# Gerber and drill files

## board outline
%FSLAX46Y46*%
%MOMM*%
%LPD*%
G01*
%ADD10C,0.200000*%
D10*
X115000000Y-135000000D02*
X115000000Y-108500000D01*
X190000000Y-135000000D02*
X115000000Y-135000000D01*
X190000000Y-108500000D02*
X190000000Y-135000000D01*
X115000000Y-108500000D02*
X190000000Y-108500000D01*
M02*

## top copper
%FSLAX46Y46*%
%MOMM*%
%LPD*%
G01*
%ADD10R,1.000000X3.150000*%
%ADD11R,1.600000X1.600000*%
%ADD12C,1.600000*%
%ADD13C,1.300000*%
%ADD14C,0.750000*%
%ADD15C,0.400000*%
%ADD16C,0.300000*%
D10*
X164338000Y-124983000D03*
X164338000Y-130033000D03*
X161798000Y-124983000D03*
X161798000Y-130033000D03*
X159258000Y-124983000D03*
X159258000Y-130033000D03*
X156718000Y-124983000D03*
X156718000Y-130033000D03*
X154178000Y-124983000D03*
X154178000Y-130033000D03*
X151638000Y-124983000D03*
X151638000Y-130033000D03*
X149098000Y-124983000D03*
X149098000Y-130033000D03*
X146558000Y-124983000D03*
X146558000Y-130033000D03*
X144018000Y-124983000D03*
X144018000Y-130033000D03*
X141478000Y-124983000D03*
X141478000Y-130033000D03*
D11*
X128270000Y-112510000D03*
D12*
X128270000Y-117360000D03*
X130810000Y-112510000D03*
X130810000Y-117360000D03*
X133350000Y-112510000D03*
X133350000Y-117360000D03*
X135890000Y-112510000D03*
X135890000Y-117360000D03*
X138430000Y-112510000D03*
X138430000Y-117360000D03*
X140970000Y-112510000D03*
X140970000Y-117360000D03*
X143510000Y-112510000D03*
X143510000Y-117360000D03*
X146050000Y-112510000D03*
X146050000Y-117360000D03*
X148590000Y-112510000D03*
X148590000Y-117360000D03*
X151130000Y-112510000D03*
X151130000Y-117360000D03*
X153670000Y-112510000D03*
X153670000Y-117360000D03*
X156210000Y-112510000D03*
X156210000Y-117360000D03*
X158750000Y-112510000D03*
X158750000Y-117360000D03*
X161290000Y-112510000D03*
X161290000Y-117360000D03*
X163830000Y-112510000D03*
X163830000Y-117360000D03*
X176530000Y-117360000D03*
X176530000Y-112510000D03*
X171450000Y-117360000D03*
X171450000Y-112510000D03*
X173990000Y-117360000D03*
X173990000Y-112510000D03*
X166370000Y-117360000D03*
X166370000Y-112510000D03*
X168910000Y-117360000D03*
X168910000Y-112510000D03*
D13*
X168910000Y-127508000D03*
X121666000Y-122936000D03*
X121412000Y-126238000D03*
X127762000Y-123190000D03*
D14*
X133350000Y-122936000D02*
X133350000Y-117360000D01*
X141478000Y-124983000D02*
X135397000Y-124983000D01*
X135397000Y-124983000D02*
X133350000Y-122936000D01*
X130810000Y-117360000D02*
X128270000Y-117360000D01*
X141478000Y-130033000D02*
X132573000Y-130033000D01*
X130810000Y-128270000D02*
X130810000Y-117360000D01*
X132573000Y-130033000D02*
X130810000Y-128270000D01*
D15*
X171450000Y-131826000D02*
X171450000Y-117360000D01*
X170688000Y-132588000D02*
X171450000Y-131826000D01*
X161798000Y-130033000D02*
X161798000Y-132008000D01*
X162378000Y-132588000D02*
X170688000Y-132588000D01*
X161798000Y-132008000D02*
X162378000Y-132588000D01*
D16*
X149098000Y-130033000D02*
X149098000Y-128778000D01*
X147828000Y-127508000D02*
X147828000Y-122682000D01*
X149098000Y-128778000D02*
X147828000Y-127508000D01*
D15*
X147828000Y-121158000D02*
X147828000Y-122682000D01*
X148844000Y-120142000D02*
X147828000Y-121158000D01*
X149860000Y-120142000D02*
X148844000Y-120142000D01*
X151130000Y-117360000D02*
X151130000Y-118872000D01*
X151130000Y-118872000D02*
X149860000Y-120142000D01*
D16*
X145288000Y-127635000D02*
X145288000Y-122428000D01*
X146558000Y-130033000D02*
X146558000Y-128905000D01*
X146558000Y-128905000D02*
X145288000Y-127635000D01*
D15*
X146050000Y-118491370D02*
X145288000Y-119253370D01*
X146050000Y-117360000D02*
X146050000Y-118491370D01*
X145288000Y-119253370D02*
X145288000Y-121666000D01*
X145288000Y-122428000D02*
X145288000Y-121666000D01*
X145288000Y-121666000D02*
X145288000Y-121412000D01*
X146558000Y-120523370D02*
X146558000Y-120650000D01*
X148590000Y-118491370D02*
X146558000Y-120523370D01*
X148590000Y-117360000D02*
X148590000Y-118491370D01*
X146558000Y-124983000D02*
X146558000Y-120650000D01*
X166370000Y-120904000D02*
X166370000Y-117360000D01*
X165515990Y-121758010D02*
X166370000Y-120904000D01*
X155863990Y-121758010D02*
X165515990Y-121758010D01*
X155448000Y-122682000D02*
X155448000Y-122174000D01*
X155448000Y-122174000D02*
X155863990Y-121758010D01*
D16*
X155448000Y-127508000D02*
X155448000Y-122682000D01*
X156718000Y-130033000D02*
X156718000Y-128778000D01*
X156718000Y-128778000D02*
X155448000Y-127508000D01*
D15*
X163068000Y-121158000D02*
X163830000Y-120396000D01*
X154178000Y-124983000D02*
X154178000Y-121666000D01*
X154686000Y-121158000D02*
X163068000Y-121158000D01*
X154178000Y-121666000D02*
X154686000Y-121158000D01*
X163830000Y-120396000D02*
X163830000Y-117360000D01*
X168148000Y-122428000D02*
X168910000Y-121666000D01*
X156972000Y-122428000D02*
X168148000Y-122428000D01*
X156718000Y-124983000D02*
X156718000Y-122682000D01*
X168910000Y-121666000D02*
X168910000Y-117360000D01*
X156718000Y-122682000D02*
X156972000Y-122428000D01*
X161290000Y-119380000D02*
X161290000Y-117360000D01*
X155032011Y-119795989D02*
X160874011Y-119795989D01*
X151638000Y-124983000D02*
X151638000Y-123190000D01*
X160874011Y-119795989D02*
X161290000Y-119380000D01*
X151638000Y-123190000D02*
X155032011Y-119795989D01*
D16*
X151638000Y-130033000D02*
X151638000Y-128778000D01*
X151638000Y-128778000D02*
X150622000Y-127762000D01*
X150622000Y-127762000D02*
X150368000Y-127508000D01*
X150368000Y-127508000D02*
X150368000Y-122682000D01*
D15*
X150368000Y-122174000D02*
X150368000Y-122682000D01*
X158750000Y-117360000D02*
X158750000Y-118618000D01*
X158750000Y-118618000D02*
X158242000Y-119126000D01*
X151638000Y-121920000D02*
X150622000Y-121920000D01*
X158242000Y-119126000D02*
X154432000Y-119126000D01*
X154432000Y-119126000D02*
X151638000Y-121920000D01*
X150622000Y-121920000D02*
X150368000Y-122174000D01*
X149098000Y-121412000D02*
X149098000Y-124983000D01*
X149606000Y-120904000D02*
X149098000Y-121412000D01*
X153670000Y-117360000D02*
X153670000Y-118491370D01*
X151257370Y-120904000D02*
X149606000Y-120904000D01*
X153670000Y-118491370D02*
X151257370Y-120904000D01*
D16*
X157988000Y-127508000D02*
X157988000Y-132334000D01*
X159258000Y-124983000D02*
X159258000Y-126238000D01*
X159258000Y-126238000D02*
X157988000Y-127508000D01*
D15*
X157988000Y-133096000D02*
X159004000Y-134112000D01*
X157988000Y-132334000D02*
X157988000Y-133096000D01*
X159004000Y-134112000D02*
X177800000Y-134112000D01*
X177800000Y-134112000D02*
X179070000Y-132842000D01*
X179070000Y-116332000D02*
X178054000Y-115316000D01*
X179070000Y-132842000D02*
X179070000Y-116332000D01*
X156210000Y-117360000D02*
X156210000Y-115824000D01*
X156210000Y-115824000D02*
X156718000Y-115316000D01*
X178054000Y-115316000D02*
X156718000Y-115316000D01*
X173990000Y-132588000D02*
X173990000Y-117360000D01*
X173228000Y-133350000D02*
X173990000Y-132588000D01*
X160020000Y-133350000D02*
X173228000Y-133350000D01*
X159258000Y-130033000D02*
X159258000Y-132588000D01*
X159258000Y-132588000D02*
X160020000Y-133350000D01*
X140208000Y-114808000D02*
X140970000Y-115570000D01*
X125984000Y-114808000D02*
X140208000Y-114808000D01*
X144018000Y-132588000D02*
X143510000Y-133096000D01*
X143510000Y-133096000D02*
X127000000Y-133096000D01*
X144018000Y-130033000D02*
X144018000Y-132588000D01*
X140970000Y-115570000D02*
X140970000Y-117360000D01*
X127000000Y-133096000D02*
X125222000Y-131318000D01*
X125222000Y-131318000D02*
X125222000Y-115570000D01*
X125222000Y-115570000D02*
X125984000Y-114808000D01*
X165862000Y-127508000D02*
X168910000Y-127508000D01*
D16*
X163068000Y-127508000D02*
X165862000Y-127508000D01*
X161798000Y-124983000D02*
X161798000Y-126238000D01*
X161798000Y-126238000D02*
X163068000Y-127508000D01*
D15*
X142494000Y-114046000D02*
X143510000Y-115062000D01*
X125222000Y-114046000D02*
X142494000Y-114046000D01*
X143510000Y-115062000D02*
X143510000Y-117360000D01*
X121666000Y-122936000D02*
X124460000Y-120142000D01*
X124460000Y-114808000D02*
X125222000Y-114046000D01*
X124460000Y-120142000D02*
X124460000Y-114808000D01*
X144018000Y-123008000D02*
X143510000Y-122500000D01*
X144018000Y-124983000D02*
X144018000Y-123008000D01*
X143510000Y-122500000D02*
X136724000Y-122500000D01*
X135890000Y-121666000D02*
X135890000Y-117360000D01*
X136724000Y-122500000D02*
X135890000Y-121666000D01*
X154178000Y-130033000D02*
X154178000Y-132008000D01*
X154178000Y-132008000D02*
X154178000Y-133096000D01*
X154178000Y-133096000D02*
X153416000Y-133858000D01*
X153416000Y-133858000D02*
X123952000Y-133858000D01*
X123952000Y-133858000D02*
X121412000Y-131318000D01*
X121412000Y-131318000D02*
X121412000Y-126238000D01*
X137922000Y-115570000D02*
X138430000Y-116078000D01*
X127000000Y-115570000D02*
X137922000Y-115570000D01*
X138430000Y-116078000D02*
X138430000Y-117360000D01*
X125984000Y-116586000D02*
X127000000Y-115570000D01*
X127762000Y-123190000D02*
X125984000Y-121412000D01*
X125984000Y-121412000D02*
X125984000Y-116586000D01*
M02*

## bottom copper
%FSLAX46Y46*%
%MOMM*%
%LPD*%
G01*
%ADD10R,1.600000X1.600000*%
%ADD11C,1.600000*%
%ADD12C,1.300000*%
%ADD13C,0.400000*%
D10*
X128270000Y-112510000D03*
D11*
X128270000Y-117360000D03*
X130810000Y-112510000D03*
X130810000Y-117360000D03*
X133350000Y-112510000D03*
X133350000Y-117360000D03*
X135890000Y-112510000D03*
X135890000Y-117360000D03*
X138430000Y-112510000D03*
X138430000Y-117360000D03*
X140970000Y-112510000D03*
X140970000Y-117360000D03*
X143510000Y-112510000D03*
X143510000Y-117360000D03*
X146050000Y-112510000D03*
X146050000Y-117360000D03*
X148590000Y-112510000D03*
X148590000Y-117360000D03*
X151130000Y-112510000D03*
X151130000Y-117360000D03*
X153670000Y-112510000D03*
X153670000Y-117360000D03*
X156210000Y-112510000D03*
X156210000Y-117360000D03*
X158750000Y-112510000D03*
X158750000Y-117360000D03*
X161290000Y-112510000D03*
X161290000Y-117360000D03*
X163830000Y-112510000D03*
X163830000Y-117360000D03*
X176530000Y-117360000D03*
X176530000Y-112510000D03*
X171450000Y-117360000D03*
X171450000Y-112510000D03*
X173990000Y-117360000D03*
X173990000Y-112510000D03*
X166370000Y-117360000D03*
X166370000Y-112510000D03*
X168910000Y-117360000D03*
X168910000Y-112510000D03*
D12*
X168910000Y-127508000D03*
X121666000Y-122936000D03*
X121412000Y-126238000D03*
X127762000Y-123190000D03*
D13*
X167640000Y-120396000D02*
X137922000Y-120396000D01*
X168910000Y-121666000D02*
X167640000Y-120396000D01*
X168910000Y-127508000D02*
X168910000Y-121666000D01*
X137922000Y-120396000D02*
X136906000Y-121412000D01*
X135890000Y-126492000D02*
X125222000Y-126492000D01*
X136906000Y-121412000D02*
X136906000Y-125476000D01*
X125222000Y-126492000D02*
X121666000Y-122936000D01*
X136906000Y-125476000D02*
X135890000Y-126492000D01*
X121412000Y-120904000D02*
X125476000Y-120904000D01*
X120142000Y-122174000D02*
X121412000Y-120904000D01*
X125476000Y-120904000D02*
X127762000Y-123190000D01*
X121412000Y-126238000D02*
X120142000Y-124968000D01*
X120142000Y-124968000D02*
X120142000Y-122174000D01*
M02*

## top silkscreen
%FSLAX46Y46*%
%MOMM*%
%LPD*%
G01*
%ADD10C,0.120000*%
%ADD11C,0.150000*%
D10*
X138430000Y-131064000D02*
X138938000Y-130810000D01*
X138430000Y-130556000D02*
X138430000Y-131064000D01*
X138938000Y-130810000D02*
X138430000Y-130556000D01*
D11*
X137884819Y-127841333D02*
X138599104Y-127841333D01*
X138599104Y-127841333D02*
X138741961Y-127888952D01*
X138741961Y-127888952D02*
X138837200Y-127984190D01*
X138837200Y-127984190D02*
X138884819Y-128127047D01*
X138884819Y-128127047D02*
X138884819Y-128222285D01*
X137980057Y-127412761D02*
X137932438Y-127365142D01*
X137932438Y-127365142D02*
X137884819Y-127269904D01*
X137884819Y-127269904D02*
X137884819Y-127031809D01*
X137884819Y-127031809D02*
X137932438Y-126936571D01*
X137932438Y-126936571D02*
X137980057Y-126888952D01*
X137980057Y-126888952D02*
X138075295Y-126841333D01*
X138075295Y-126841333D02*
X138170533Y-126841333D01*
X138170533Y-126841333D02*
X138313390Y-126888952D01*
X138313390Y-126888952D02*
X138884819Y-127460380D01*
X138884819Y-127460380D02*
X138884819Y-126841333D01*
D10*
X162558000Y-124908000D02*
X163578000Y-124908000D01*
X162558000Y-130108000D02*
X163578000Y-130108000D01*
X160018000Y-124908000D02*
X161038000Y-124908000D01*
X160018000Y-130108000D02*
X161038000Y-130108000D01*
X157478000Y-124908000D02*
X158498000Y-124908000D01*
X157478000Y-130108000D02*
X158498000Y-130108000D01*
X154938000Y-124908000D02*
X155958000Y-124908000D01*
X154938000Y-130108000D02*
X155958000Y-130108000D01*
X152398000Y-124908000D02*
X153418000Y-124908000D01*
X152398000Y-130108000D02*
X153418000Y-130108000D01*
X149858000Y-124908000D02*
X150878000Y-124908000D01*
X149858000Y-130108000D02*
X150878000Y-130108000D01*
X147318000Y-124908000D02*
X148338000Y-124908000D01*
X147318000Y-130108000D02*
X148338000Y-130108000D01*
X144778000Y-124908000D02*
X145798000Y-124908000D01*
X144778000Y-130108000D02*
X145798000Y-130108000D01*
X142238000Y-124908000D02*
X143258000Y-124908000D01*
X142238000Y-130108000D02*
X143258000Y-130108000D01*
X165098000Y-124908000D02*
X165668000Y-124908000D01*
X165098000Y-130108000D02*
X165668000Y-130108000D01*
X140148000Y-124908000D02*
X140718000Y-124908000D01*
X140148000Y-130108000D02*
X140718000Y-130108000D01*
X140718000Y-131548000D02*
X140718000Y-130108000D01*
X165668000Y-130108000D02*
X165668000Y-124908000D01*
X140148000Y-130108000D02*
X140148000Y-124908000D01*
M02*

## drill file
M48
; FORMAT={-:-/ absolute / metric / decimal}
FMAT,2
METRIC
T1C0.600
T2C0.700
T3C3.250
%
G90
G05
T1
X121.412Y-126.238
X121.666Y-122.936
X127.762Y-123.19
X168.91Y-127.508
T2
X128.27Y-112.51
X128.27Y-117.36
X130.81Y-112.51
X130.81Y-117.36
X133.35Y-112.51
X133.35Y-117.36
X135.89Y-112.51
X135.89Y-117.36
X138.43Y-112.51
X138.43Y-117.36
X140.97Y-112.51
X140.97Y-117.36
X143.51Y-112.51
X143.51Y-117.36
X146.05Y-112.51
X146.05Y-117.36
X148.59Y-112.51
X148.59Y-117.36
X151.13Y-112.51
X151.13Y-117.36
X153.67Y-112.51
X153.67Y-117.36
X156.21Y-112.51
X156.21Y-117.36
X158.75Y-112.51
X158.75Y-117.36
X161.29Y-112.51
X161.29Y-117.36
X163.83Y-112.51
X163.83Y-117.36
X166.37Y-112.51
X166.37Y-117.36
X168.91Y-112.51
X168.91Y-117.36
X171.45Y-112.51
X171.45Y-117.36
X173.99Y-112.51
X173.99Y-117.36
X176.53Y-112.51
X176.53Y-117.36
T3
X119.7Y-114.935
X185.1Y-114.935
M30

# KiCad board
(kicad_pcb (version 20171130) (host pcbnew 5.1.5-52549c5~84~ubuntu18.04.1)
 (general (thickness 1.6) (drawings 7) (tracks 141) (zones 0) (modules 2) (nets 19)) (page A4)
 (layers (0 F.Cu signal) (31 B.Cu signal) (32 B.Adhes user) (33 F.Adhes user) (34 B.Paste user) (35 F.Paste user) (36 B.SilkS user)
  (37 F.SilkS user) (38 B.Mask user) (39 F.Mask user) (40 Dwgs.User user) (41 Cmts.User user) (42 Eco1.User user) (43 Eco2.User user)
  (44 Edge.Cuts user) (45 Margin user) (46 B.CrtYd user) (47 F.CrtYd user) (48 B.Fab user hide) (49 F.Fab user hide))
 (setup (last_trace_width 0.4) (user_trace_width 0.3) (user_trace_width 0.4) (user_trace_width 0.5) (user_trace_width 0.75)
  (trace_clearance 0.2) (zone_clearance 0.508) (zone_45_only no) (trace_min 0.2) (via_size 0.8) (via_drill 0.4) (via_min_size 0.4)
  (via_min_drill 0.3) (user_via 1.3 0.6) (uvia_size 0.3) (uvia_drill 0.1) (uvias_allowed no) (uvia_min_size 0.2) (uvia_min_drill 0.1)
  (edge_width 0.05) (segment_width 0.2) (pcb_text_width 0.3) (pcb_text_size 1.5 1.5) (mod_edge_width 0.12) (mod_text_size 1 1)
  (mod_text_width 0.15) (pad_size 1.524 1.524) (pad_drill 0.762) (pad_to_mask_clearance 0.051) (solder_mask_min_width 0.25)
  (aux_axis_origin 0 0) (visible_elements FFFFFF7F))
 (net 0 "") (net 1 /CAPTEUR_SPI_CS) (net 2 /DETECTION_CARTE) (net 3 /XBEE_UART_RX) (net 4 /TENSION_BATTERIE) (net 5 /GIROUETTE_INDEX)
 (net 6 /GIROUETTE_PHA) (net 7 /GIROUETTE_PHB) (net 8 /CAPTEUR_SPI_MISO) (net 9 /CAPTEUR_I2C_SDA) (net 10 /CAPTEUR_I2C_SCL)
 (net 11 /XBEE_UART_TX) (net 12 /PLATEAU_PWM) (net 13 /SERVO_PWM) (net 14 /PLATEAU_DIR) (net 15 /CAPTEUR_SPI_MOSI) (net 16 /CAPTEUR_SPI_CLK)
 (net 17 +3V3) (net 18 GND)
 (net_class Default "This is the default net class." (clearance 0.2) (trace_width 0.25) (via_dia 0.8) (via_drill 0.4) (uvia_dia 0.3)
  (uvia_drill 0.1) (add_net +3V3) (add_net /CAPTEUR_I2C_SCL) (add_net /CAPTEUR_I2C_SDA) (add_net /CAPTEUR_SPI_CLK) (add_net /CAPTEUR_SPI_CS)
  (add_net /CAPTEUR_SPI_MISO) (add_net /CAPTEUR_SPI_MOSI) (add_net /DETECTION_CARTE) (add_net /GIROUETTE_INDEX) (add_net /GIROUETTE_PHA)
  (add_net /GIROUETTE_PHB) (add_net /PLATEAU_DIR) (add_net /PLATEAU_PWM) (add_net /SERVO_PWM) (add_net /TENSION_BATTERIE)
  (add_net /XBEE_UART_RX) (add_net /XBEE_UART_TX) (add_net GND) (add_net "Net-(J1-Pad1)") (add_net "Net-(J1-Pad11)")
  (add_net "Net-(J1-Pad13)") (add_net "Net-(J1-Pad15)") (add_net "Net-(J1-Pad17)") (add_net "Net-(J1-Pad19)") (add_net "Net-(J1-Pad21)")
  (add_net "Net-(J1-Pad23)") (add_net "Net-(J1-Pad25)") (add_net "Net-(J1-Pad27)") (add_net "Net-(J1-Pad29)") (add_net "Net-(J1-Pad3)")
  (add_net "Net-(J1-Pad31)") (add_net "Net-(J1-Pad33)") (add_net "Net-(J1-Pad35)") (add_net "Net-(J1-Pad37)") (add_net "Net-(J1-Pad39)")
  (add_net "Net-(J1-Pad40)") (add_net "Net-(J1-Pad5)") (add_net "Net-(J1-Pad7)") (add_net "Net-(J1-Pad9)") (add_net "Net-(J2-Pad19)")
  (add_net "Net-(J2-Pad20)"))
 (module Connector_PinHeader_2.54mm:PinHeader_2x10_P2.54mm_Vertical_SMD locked (layer F.Cu) (at 152.908 127.508 90)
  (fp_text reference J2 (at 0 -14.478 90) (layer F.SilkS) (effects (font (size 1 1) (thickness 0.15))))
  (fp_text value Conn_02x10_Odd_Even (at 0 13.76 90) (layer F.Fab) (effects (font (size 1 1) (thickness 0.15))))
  (fp_line (start 2.6 9.65) (end 2.6 10.67) (layer F.SilkS) (width 0.12))
  (fp_line (start -2.6 9.65) (end -2.6 10.67) (layer F.SilkS) (width 0.12))
  (fp_line (start 2.6 7.11) (end 2.6 8.13) (layer F.SilkS) (width 0.12))
  (fp_line (start -2.6 7.11) (end -2.6 8.13) (layer F.SilkS) (width 0.12))
  (fp_line (start 2.6 4.57) (end 2.6 5.59) (layer F.SilkS) (width 0.12))
  (fp_line (start -2.6 4.57) (end -2.6 5.59) (layer F.SilkS) (width 0.12))
  (fp_line (start 2.6 2.03) (end 2.6 3.05) (layer F.SilkS) (width 0.12))
  (fp_line (start -2.6 2.03) (end -2.6 3.05) (layer F.SilkS) (width 0.12))
  (fp_line (start 2.6 -0.51) (end 2.6 0.51) (layer F.SilkS) (width 0.12))
  (fp_line (start -2.6 -0.51) (end -2.6 0.51) (layer F.SilkS) (width 0.12))
  (fp_line (start 2.6 -3.05) (end 2.6 -2.03) (layer F.SilkS) (width 0.12))
  (fp_line (start -2.6 -3.05) (end -2.6 -2.03) (layer F.SilkS) (width 0.12))
  (fp_line (start 2.6 -5.59) (end 2.6 -4.57) (layer F.SilkS) (width 0.12))
  (fp_line (start -2.6 -5.59) (end -2.6 -4.57) (layer F.SilkS) (width 0.12))
  (fp_line (start 2.6 -8.13) (end 2.6 -7.11) (layer F.SilkS) (width 0.12))
  (fp_line (start -2.6 -8.13) (end -2.6 -7.11) (layer F.SilkS) (width 0.12))
  (fp_line (start 2.6 -10.67) (end 2.6 -9.65) (layer F.SilkS) (width 0.12))
  (fp_line (start -2.6 -10.67) (end -2.6 -9.65) (layer F.SilkS) (width 0.12))
  (fp_line (start 2.6 12.19) (end 2.6 12.76) (layer F.SilkS) (width 0.12))
  (fp_line (start -2.6 12.19) (end -2.6 12.76) (layer F.SilkS) (width 0.12))
  (fp_line (start 2.6 -12.76) (end 2.6 -12.19) (layer F.SilkS) (width 0.12))
  (fp_line (start -2.6 -12.76) (end -2.6 -12.19) (layer F.SilkS) (width 0.12))
  (fp_line (start -4.04 -12.19) (end -2.6 -12.19) (layer F.SilkS) (width 0.12))
  (fp_line (start -2.6 12.76) (end 2.6 12.76) (layer F.SilkS) (width 0.12))
  (fp_line (start -2.6 -12.76) (end 2.6 -12.76) (layer F.SilkS) (width 0.12))
  (pad 20 smd rect (at 2.525 11.43 90) (size 3.15 1) (layers F.Cu F.Paste F.Mask))
  (pad 19 smd rect (at -2.525 11.43 90) (size 3.15 1) (layers F.Cu F.Paste F.Mask))
  (pad 18 smd rect (at 2.525 8.89 90) (size 3.15 1) (layers F.Cu F.Paste F.Mask) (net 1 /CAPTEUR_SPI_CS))
  (pad 17 smd rect (at -2.525 8.89 90) (size 3.15 1) (layers F.Cu F.Paste F.Mask) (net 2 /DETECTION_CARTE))
  (pad 16 smd rect (at 2.525 6.35 90) (size 3.15 1) (layers F.Cu F.Paste F.Mask) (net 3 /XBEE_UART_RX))
  (pad 15 smd rect (at -2.525 6.35 90) (size 3.15 1) (layers F.Cu F.Paste F.Mask) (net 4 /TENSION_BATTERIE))
  (pad 14 smd rect (at 2.525 3.81 90) (size 3.15 1) (layers F.Cu F.Paste F.Mask) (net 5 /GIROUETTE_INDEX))
  (pad 13 smd rect (at -2.525 3.81 90) (size 3.15 1) (layers F.Cu F.Paste F.Mask) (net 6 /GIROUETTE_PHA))
  (pad 12 smd rect (at 2.525 1.27 90) (size 3.15 1) (layers F.Cu F.Paste F.Mask) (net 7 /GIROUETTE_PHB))
  (pad 11 smd rect (at -2.525 1.27 90) (size 3.15 1) (layers F.Cu F.Paste F.Mask) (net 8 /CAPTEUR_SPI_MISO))
  (pad 10 smd rect (at 2.525 -1.27 90) (size 3.15 1) (layers F.Cu F.Paste F.Mask) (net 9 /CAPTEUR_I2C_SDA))
  (pad 9 smd rect (at -2.525 -1.27 90) (size 3.15 1) (layers F.Cu F.Paste F.Mask) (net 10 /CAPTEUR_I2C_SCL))
  (pad 8 smd rect (at 2.525 -3.81 90) (size 3.15 1) (layers F.Cu F.Paste F.Mask) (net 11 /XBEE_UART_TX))
  (pad 7 smd rect (at -2.525 -3.81 90) (size 3.15 1) (layers F.Cu F.Paste F.Mask) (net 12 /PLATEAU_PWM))
  (pad 6 smd rect (at 2.525 -6.35 90) (size 3.15 1) (layers F.Cu F.Paste F.Mask) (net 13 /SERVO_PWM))
  (pad 5 smd rect (at -2.525 -6.35 90) (size 3.15 1) (layers F.Cu F.Paste F.Mask) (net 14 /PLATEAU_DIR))
  (pad 4 smd rect (at 2.525 -8.89 90) (size 3.15 1) (layers F.Cu F.Paste F.Mask) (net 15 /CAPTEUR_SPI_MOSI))
  (pad 3 smd rect (at -2.525 -8.89 90) (size 3.15 1) (layers F.Cu F.Paste F.Mask) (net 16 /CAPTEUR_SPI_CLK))
  (pad 2 smd rect (at 2.525 -11.43 90) (size 3.15 1) (layers F.Cu F.Paste F.Mask) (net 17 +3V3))
  (pad 1 smd rect (at -2.525 -11.43 90) (size 3.15 1) (layers F.Cu F.Paste F.Mask) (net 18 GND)))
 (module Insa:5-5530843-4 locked (layer B.Cu) (at 146.05 114.935)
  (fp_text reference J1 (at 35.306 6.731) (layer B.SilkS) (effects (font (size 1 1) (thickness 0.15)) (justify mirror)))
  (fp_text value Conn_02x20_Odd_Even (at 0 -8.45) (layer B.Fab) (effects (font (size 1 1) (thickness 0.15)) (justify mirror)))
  (pad 1 thru_hole rect (at -17.78 -2.425) (size 1.6 1.6) (drill 0.7) (layers *.Cu *.Mask))
  (pad 2 thru_hole circle (at -17.78 2.425) (size 1.6 1.6) (drill 0.7) (layers *.Cu *.Mask) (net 18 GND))
  (pad 3 thru_hole circle (at -15.24 -2.425) (size 1.6 1.6) (drill 0.7) (layers *.Cu *.Mask))
  (pad 4 thru_hole circle (at -15.24 2.425) (size 1.6 1.6) (drill 0.7) (layers *.Cu *.Mask) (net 18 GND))
  (pad 5 thru_hole circle (at -12.7 -2.425) (size 1.6 1.6) (drill 0.7) (layers *.Cu *.Mask))
  (pad 6 thru_hole circle (at -12.7 2.425) (size 1.6 1.6) (drill 0.7) (layers *.Cu *.Mask) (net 17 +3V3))
  (pad 7 thru_hole circle (at -10.16 -2.425) (size 1.6 1.6) (drill 0.7) (layers *.Cu *.Mask))
  (pad 8 thru_hole circle (at -10.16 2.425) (size 1.6 1.6) (drill 0.7) (layers *.Cu *.Mask) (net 15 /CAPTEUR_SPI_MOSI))
  (pad 9 thru_hole circle (at -7.62 -2.425) (size 1.6 1.6) (drill 0.7) (layers *.Cu *.Mask))
  (pad 10 thru_hole circle (at -7.62 2.425) (size 1.6 1.6) (drill 0.7) (layers *.Cu *.Mask) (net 8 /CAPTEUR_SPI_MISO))
  (pad 11 thru_hole circle (at -5.08 -2.425) (size 1.6 1.6) (drill 0.7) (layers *.Cu *.Mask))
  (pad 12 thru_hole circle (at -5.08 2.425) (size 1.6 1.6) (drill 0.7) (layers *.Cu *.Mask) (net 16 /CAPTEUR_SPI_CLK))
  (pad 13 thru_hole circle (at -2.54 -2.425) (size 1.6 1.6) (drill 0.7) (layers *.Cu *.Mask))
  (pad 14 thru_hole circle (at -2.54 2.425) (size 1.6 1.6) (drill 0.7) (layers *.Cu *.Mask) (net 1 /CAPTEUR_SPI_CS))
  (pad 15 thru_hole circle (at 0 -2.425) (size 1.6 1.6) (drill 0.7) (layers *.Cu *.Mask))
  (pad 16 thru_hole circle (at 0 2.425) (size 1.6 1.6) (drill 0.7) (layers *.Cu *.Mask) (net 14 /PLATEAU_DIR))
  (pad 17 thru_hole circle (at 2.54 -2.425) (size 1.6 1.6) (drill 0.7) (layers *.Cu *.Mask))
  (pad 18 thru_hole circle (at 2.54 2.425) (size 1.6 1.6) (drill 0.7) (layers *.Cu *.Mask) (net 13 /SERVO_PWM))
  (pad 19 thru_hole circle (at 5.08 -2.425) (size 1.6 1.6) (drill 0.7) (layers *.Cu *.Mask))
  (pad 20 thru_hole circle (at 5.08 2.425) (size 1.6 1.6) (drill 0.7) (layers *.Cu *.Mask) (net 12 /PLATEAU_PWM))
  (pad 21 thru_hole circle (at 7.62 -2.425) (size 1.6 1.6) (drill 0.7) (layers *.Cu *.Mask))
  (pad 22 thru_hole circle (at 7.62 2.425) (size 1.6 1.6) (drill 0.7) (layers *.Cu *.Mask) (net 11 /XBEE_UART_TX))
  (pad 23 thru_hole circle (at 10.16 -2.425) (size 1.6 1.6) (drill 0.7) (layers *.Cu *.Mask))
  (pad 24 thru_hole circle (at 10.16 2.425) (size 1.6 1.6) (drill 0.7) (layers *.Cu *.Mask) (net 3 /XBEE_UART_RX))
  (pad 25 thru_hole circle (at 12.7 -2.425) (size 1.6 1.6) (drill 0.7) (layers *.Cu *.Mask))
  (pad 26 thru_hole circle (at 12.7 2.425) (size 1.6 1.6) (drill 0.7) (layers *.Cu *.Mask) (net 10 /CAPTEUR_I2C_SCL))
  (pad 27 thru_hole circle (at 15.24 -2.425) (size 1.6 1.6) (drill 0.7) (layers *.Cu *.Mask))
  (pad 28 thru_hole circle (at 15.24 2.425) (size 1.6 1.6) (drill 0.7) (layers *.Cu *.Mask) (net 9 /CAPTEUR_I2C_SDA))
  (pad 29 thru_hole circle (at 17.78 -2.425) (size 1.6 1.6) (drill 0.7) (layers *.Cu *.Mask))
  (pad 30 thru_hole circle (at 17.78 2.425) (size 1.6 1.6) (drill 0.7) (layers *.Cu *.Mask) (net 7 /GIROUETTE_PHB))
  (pad "" np_thru_hole circle (at 39.05 0) (size 3.25 3.25) (drill 3.25) (layers *.Cu *.Mask))
  (pad "" np_thru_hole circle (at -26.35 0) (size 3.25 3.25) (drill 3.25) (layers *.Cu *.Mask))
  (pad 40 thru_hole circle (at 30.48 2.425) (size 1.6 1.6) (drill 0.7) (layers *.Cu *.Mask))
  (pad 39 thru_hole circle (at 30.48 -2.425) (size 1.6 1.6) (drill 0.7) (layers *.Cu *.Mask))
  (pad 36 thru_hole circle (at 25.4 2.425) (size 1.6 1.6) (drill 0.7) (layers *.Cu *.Mask) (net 2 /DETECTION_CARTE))
  (pad 35 thru_hole circle (at 25.4 -2.425) (size 1.6 1.6) (drill 0.7) (layers *.Cu *.Mask))
  (pad 38 thru_hole circle (at 27.94 2.425) (size 1.6 1.6) (drill 0.7) (layers *.Cu *.Mask) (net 4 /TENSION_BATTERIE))
  (pad 37 thru_hole circle (at 27.94 -2.425) (size 1.6 1.6) (drill 0.7) (layers *.Cu *.Mask))
  (pad 32 thru_hole circle (at 20.32 2.425) (size 1.6 1.6) (drill 0.7) (layers *.Cu *.Mask) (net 6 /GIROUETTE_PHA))
  (pad 31 thru_hole circle (at 20.32 -2.425) (size 1.6 1.6) (drill 0.7) (layers *.Cu *.Mask))
  (pad 34 thru_hole circle (at 22.86 2.425) (size 1.6 1.6) (drill 0.7) (layers *.Cu *.Mask) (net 5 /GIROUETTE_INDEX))
  (pad 33 thru_hole circle (at 22.86 -2.425) (size 1.6 1.6) (drill 0.7) (layers *.Cu *.Mask)))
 (gr_line (start 138.43 131.064) (end 138.938 130.81) (layer F.SilkS) (width 0.12))
 (gr_line (start 138.43 130.556) (end 138.43 131.064) (layer F.SilkS) (width 0.12))
 (gr_line (start 138.938 130.81) (end 138.43 130.556) (layer F.SilkS) (width 0.12))
 (gr_line (start 115 135) (end 115 108.5) (layer Edge.Cuts) (width 0.2))
 (gr_line (start 190 135) (end 115 135) (layer Edge.Cuts) (width 0.2))
 (gr_line (start 190 108.5) (end 190 135) (layer Edge.Cuts) (width 0.2))
 (gr_line (start 115 108.5) (end 190 108.5) (layer Edge.Cuts) (width 0.2))
 (segment (start 133.35 122.936) (end 133.35 117.36) (width 0.75) (layer F.Cu) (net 17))
 (segment (start 141.478 124.983) (end 135.397 124.983) (width 0.75) (layer F.Cu) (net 17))
 (segment (start 135.397 124.983) (end 133.35 122.936) (width 0.75) (layer F.Cu) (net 17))
 (segment (start 130.81 117.36) (end 128.27 117.36) (width 0.75) (layer F.Cu) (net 18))
 (segment (start 141.478 130.033) (end 132.573 130.033) (width 0.75) (layer F.Cu) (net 18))
 (segment (start 130.81 128.27) (end 130.81 117.36) (width 0.75) (layer F.Cu) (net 18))
 (segment (start 132.573 130.033) (end 130.81 128.27) (width 0.75) (layer F.Cu) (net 18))
 (segment (start 171.45 131.826) (end 171.45 117.36) (width 0.4) (layer F.Cu) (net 2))
 (segment (start 170.688 132.588) (end 171.45 131.826) (width 0.4) (layer F.Cu) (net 2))
 (segment (start 161.798 130.033) (end 161.798 132.008) (width 0.4) (layer F.Cu) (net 2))
 (segment (start 162.378 132.588) (end 170.688 132.588) (width 0.4) (layer F.Cu) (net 2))
 (segment (start 161.798 132.008) (end 162.378 132.588) (width 0.4) (layer F.Cu) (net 2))
 (segment (start 149.098 130.033) (end 149.098 128.778) (width 0.3) (layer F.Cu) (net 12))
 (segment (start 147.828 127.508) (end 147.828 122.682) (width 0.3) (layer F.Cu) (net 12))
 (segment (start 149.098 128.778) (end 147.828 127.508) (width 0.3) (layer F.Cu) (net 12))
 (segment (start 147.828 121.158) (end 147.828 122.682) (width 0.4) (layer F.Cu) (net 12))
 (segment (start 148.844 120.142) (end 147.828 121.158) (width 0.4) (layer F.Cu) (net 12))
 (segment (start 149.86 120.142) (end 148.844 120.142) (width 0.4) (layer F.Cu) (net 12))
 (segment (start 151.13 117.36) (end 151.13 118.872) (width 0.4) (layer F.Cu) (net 12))
 (segment (start 151.13 118.872) (end 149.86 120.142) (width 0.4) (layer F.Cu) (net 12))
 (segment (start 145.288 127.635) (end 145.288 122.428) (width 0.3) (layer F.Cu) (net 14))
 (segment (start 146.558 130.033) (end 146.558 128.905) (width 0.3) (layer F.Cu) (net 14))
 (segment (start 146.558 128.905) (end 145.288 127.635) (width 0.3) (layer F.Cu) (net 14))
 (segment (start 146.05 118.49137) (end 145.288 119.25337) (width 0.4) (layer F.Cu) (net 14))
 (segment (start 146.05 117.36) (end 146.05 118.49137) (width 0.4) (layer F.Cu) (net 14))
 (segment (start 145.288 119.25337) (end 145.288 121.666) (width 0.4) (layer F.Cu) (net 14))
 (segment (start 145.288 122.428) (end 145.288 121.666) (width 0.4) (layer F.Cu) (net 14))
 (segment (start 145.288 121.666) (end 145.288 121.412) (width 0.4) (layer F.Cu) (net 14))
 (segment (start 146.558 120.52337) (end 146.558 120.65) (width 0.4) (layer F.Cu) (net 13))
 (segment (start 148.59 118.49137) (end 146.558 120.52337) (width 0.4) (layer F.Cu) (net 13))
 (segment (start 148.59 117.36) (end 148.59 118.49137) (width 0.4) (layer F.Cu) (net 13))
 (segment (start 146.558 124.983) (end 146.558 120.65) (width 0.4) (layer F.Cu) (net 13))
 (segment (start 166.37 120.904) (end 166.37 117.36) (width 0.4) (layer F.Cu) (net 6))
 (segment (start 165.51599 121.75801) (end 166.37 120.904) (width 0.4) (layer F.Cu) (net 6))
 (segment (start 155.86399 121.75801) (end 165.51599 121.75801) (width 0.4) (layer F.Cu) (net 6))
 (segment (start 155.448 122.682) (end 155.448 122.174) (width 0.4) (layer F.Cu) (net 6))
 (segment (start 155.448 122.174) (end 155.86399 121.75801) (width 0.4) (layer F.Cu) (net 6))
 (segment (start 155.448 127.508) (end 155.448 122.682) (width 0.3) (layer F.Cu) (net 6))
 (segment (start 156.718 130.033) (end 156.718 128.778) (width 0.3) (layer F.Cu) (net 6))
 (segment (start 156.718 128.778) (end 155.448 127.508) (width 0.3) (layer F.Cu) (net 6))
 (segment (start 163.068 121.158) (end 163.83 120.396) (width 0.4) (layer F.Cu) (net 7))
 (segment (start 154.178 124.983) (end 154.178 121.666) (width 0.4) (layer F.Cu) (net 7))
 (segment (start 154.686 121.158) (end 163.068 121.158) (width 0.4) (layer F.Cu) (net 7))
 (segment (start 154.178 121.666) (end 154.686 121.158) (width 0.4) (layer F.Cu) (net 7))
 (segment (start 163.83 120.396) (end 163.83 117.36) (width 0.4) (layer F.Cu) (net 7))
 (segment (start 168.148 122.428) (end 168.91 121.666) (width 0.4) (layer F.Cu) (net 5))
 (segment (start 156.972 122.428) (end 168.148 122.428) (width 0.4) (layer F.Cu) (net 5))
 (segment (start 156.718 124.983) (end 156.718 122.682) (width 0.4) (layer F.Cu) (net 5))
 (segment (start 168.91 121.666) (end 168.91 117.36) (width 0.4) (layer F.Cu) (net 5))
 (segment (start 156.718 122.682) (end 156.972 122.428) (width 0.4) (layer F.Cu) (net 5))
 (segment (start 161.29 119.38) (end 161.29 117.36) (width 0.4) (layer F.Cu) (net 9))
 (segment (start 155.032011 119.795989) (end 160.874011 119.795989) (width 0.4) (layer F.Cu) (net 9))
 (segment (start 151.638 124.983) (end 151.638 123.19) (width 0.4) (layer F.Cu) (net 9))
 (segment (start 160.874011 119.795989) (end 161.29 119.38) (width 0.4) (layer F.Cu) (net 9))
 (segment (start 151.638 123.19) (end 155.032011 119.795989) (width 0.4) (layer F.Cu) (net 9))
 (segment (start 151.638 130.033) (end 151.638 128.778) (width 0.3) (layer F.Cu) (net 10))
 (segment (start 151.638 128.778) (end 150.622 127.762) (width 0.3) (layer F.Cu) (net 10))
 (segment (start 150.622 127.762) (end 150.368 127.508) (width 0.3) (layer F.Cu) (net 10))
 (segment (start 150.368 127.508) (end 150.368 122.682) (width 0.3) (layer F.Cu) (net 10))
 (segment (start 150.368 122.174) (end 150.368 122.682) (width 0.4) (layer F.Cu) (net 10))
 (segment (start 158.75 117.36) (end 158.75 118.618) (width 0.4) (layer F.Cu) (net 10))
 (segment (start 158.75 118.618) (end 158.242 119.126) (width 0.4) (layer F.Cu) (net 10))
 (segment (start 151.638 121.92) (end 150.622 121.92) (width 0.4) (layer F.Cu) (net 10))
 (segment (start 158.242 119.126) (end 154.432 119.126) (width 0.4) (layer F.Cu) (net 10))
 (segment (start 154.432 119.126) (end 151.638 121.92) (width 0.4) (layer F.Cu) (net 10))
 (segment (start 150.622 121.92) (end 150.368 122.174) (width 0.4) (layer F.Cu) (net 10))
 (segment (start 149.098 121.412) (end 149.098 124.983) (width 0.4) (layer F.Cu) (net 11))
 (segment (start 149.606 120.904) (end 149.098 121.412) (width 0.4) (layer F.Cu) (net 11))
 (segment (start 153.67 117.36) (end 153.67 118.49137) (width 0.4) (layer F.Cu) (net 11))
 (segment (start 151.25737 120.904) (end 149.606 120.904) (width 0.4) (layer F.Cu) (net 11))
 (segment (start 153.67 118.49137) (end 151.25737 120.904) (width 0.4) (layer F.Cu) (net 11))
 (segment (start 157.988 127.508) (end 157.988 132.334) (width 0.3) (layer F.Cu) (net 3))
 (segment (start 159.258 124.983) (end 159.258 126.238) (width 0.3) (layer F.Cu) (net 3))
 (segment (start 159.258 126.238) (end 157.988 127.508) (width 0.3) (layer F.Cu) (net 3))
 (segment (start 157.988 133.096) (end 159.004 134.112) (width 0.4) (layer F.Cu) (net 3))
 (segment (start 157.988 132.334) (end 157.988 133.096) (width 0.4) (layer F.Cu) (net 3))
 (segment (start 159.004 134.112) (end 177.8 134.112) (width 0.4) (layer F.Cu) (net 3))
 (segment (start 177.8 134.112) (end 179.07 132.842) (width 0.4) (layer F.Cu) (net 3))
 (segment (start 179.07 116.332) (end 178.054 115.316) (width 0.4) (layer F.Cu) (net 3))
 (segment (start 179.07 132.842) (end 179.07 116.332) (width 0.4) (layer F.Cu) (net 3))
 (segment (start 156.21 117.36) (end 156.21 115.824) (width 0.4) (layer F.Cu) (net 3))
 (segment (start 156.21 115.824) (end 156.718 115.316) (width 0.4) (layer F.Cu) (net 3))
 (segment (start 178.054 115.316) (end 156.718 115.316) (width 0.4) (layer F.Cu) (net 3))
 (segment (start 173.99 132.588) (end 173.99 117.36) (width 0.4) (layer F.Cu) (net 4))
 (segment (start 173.228 133.35) (end 173.99 132.588) (width 0.4) (layer F.Cu) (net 4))
 (segment (start 160.02 133.35) (end 173.228 133.35) (width 0.4) (layer F.Cu) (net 4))
 (segment (start 159.258 130.033) (end 159.258 132.588) (width 0.4) (layer F.Cu) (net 4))
 (segment (start 159.258 132.588) (end 160.02 133.35) (width 0.4) (layer F.Cu) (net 4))
 (segment (start 140.208 114.808) (end 140.97 115.57) (width 0.4) (layer F.Cu) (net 16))
 (segment (start 125.984 114.808) (end 140.208 114.808) (width 0.4) (layer F.Cu) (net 16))
 (segment (start 144.018 132.588) (end 143.51 133.096) (width 0.4) (layer F.Cu) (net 16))
 (segment (start 143.51 133.096) (end 127 133.096) (width 0.4) (layer F.Cu) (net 16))
 (segment (start 144.018 130.033) (end 144.018 132.588) (width 0.4) (layer F.Cu) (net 16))
 (segment (start 140.97 115.57) (end 140.97 117.36) (width 0.4) (layer F.Cu) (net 16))
 (segment (start 127 133.096) (end 125.222 131.318) (width 0.4) (layer F.Cu) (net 16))
 (segment (start 125.222 131.318) (end 125.222 115.57) (width 0.4) (layer F.Cu) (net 16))
 (segment (start 125.222 115.57) (end 125.984 114.808) (width 0.4) (layer F.Cu) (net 16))
 (segment (start 165.862 127.508) (end 168.91 127.508) (width 0.4) (layer F.Cu) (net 1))
 (via (at 168.91 127.508) (size 1.3) (drill 0.6) (layers F.Cu B.Cu) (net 1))
 (via (at 121.666 122.936) (size 1.3) (drill 0.6) (layers F.Cu B.Cu) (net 1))
 (segment (start 163.068 127.508) (end 165.862 127.508) (width 0.3) (layer F.Cu) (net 1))
 (segment (start 161.798 124.983) (end 161.798 126.238) (width 0.3) (layer F.Cu) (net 1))
 (segment (start 161.798 126.238) (end 163.068 127.508) (width 0.3) (layer F.Cu) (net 1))
 (segment (start 167.64 120.396) (end 137.922 120.396) (width 0.4) (layer B.Cu) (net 1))
 (segment (start 168.91 121.666) (end 167.64 120.396) (width 0.4) (layer B.Cu) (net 1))
 (segment (start 168.91 127.508) (end 168.91 121.666) (width 0.4) (layer B.Cu) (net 1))
 (segment (start 137.922 120.396) (end 136.906 121.412) (width 0.4) (layer B.Cu) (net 1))
 (segment (start 135.89 126.492) (end 125.222 126.492) (width 0.4) (layer B.Cu) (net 1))
 (segment (start 136.906 121.412) (end 136.906 125.476) (width 0.4) (layer B.Cu) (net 1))
 (segment (start 125.222 126.492) (end 121.666 122.936) (width 0.4) (layer B.Cu) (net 1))
 (segment (start 136.906 125.476) (end 135.89 126.492) (width 0.4) (layer B.Cu) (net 1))
 (segment (start 142.494 114.046) (end 143.51 115.062) (width 0.4) (layer F.Cu) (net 1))
 (segment (start 125.222 114.046) (end 142.494 114.046) (width 0.4) (layer F.Cu) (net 1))
 (segment (start 143.51 115.062) (end 143.51 117.36) (width 0.4) (layer F.Cu) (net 1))
 (segment (start 121.666 122.936) (end 124.46 120.142) (width 0.4) (layer F.Cu) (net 1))
 (segment (start 124.46 114.808) (end 125.222 114.046) (width 0.4) (layer F.Cu) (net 1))
 (segment (start 124.46 120.142) (end 124.46 114.808) (width 0.4) (layer F.Cu) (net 1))
 (segment (start 144.018 123.008) (end 143.51 122.5) (width 0.4) (layer F.Cu) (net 15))
 (segment (start 144.018 124.983) (end 144.018 123.008) (width 0.4) (layer F.Cu) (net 15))
 (segment (start 143.51 122.5) (end 136.724 122.5) (width 0.4) (layer F.Cu) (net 15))
 (segment (start 135.89 121.666) (end 135.89 117.36) (width 0.4) (layer F.Cu) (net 15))
 (segment (start 136.724 122.5) (end 135.89 121.666) (width 0.4) (layer F.Cu) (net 15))
 (segment (start 154.178 130.033) (end 154.178 132.008) (width 0.4) (layer F.Cu) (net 8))
 (segment (start 154.178 132.008) (end 154.178 133.096) (width 0.4) (layer F.Cu) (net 8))
 (segment (start 154.178 133.096) (end 153.416 133.858) (width 0.4) (layer F.Cu) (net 8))
 (segment (start 153.416 133.858) (end 123.952 133.858) (width 0.4) (layer F.Cu) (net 8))
 (via (at 121.412 126.238) (size 1.3) (drill 0.6) (layers F.Cu B.Cu) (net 8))
 (segment (start 123.952 133.858) (end 121.412 131.318) (width 0.4) (layer F.Cu) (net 8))
 (segment (start 121.412 131.318) (end 121.412 126.238) (width 0.4) (layer F.Cu) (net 8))
 (via (at 127.762 123.19) (size 1.3) (drill 0.6) (layers F.Cu B.Cu) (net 8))
 (segment (start 121.412 120.904) (end 125.476 120.904) (width 0.4) (layer B.Cu) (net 8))
 (segment (start 120.142 122.174) (end 121.412 120.904) (width 0.4) (layer B.Cu) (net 8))
 (segment (start 125.476 120.904) (end 127.762 123.19) (width 0.4) (layer B.Cu) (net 8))
 (segment (start 121.412 126.238) (end 120.142 124.968) (width 0.4) (layer B.Cu) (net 8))
 (segment (start 120.142 124.968) (end 120.142 122.174) (width 0.4) (layer B.Cu) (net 8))
 (segment (start 137.922 115.57) (end 138.43 116.078) (width 0.4) (layer F.Cu) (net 8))
 (segment (start 127 115.57) (end 137.922 115.57) (width 0.4) (layer F.Cu) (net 8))
 (segment (start 138.43 116.078) (end 138.43 117.36) (width 0.4) (layer F.Cu) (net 8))
 (segment (start 125.984 116.586) (end 127 115.57) (width 0.4) (layer F.Cu) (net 8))
 (segment (start 127.762 123.19) (end 125.984 121.412) (width 0.4) (layer F.Cu) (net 8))
 (segment (start 125.984 121.412) (end 125.984 116.586) (width 0.4) (layer F.Cu) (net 8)))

